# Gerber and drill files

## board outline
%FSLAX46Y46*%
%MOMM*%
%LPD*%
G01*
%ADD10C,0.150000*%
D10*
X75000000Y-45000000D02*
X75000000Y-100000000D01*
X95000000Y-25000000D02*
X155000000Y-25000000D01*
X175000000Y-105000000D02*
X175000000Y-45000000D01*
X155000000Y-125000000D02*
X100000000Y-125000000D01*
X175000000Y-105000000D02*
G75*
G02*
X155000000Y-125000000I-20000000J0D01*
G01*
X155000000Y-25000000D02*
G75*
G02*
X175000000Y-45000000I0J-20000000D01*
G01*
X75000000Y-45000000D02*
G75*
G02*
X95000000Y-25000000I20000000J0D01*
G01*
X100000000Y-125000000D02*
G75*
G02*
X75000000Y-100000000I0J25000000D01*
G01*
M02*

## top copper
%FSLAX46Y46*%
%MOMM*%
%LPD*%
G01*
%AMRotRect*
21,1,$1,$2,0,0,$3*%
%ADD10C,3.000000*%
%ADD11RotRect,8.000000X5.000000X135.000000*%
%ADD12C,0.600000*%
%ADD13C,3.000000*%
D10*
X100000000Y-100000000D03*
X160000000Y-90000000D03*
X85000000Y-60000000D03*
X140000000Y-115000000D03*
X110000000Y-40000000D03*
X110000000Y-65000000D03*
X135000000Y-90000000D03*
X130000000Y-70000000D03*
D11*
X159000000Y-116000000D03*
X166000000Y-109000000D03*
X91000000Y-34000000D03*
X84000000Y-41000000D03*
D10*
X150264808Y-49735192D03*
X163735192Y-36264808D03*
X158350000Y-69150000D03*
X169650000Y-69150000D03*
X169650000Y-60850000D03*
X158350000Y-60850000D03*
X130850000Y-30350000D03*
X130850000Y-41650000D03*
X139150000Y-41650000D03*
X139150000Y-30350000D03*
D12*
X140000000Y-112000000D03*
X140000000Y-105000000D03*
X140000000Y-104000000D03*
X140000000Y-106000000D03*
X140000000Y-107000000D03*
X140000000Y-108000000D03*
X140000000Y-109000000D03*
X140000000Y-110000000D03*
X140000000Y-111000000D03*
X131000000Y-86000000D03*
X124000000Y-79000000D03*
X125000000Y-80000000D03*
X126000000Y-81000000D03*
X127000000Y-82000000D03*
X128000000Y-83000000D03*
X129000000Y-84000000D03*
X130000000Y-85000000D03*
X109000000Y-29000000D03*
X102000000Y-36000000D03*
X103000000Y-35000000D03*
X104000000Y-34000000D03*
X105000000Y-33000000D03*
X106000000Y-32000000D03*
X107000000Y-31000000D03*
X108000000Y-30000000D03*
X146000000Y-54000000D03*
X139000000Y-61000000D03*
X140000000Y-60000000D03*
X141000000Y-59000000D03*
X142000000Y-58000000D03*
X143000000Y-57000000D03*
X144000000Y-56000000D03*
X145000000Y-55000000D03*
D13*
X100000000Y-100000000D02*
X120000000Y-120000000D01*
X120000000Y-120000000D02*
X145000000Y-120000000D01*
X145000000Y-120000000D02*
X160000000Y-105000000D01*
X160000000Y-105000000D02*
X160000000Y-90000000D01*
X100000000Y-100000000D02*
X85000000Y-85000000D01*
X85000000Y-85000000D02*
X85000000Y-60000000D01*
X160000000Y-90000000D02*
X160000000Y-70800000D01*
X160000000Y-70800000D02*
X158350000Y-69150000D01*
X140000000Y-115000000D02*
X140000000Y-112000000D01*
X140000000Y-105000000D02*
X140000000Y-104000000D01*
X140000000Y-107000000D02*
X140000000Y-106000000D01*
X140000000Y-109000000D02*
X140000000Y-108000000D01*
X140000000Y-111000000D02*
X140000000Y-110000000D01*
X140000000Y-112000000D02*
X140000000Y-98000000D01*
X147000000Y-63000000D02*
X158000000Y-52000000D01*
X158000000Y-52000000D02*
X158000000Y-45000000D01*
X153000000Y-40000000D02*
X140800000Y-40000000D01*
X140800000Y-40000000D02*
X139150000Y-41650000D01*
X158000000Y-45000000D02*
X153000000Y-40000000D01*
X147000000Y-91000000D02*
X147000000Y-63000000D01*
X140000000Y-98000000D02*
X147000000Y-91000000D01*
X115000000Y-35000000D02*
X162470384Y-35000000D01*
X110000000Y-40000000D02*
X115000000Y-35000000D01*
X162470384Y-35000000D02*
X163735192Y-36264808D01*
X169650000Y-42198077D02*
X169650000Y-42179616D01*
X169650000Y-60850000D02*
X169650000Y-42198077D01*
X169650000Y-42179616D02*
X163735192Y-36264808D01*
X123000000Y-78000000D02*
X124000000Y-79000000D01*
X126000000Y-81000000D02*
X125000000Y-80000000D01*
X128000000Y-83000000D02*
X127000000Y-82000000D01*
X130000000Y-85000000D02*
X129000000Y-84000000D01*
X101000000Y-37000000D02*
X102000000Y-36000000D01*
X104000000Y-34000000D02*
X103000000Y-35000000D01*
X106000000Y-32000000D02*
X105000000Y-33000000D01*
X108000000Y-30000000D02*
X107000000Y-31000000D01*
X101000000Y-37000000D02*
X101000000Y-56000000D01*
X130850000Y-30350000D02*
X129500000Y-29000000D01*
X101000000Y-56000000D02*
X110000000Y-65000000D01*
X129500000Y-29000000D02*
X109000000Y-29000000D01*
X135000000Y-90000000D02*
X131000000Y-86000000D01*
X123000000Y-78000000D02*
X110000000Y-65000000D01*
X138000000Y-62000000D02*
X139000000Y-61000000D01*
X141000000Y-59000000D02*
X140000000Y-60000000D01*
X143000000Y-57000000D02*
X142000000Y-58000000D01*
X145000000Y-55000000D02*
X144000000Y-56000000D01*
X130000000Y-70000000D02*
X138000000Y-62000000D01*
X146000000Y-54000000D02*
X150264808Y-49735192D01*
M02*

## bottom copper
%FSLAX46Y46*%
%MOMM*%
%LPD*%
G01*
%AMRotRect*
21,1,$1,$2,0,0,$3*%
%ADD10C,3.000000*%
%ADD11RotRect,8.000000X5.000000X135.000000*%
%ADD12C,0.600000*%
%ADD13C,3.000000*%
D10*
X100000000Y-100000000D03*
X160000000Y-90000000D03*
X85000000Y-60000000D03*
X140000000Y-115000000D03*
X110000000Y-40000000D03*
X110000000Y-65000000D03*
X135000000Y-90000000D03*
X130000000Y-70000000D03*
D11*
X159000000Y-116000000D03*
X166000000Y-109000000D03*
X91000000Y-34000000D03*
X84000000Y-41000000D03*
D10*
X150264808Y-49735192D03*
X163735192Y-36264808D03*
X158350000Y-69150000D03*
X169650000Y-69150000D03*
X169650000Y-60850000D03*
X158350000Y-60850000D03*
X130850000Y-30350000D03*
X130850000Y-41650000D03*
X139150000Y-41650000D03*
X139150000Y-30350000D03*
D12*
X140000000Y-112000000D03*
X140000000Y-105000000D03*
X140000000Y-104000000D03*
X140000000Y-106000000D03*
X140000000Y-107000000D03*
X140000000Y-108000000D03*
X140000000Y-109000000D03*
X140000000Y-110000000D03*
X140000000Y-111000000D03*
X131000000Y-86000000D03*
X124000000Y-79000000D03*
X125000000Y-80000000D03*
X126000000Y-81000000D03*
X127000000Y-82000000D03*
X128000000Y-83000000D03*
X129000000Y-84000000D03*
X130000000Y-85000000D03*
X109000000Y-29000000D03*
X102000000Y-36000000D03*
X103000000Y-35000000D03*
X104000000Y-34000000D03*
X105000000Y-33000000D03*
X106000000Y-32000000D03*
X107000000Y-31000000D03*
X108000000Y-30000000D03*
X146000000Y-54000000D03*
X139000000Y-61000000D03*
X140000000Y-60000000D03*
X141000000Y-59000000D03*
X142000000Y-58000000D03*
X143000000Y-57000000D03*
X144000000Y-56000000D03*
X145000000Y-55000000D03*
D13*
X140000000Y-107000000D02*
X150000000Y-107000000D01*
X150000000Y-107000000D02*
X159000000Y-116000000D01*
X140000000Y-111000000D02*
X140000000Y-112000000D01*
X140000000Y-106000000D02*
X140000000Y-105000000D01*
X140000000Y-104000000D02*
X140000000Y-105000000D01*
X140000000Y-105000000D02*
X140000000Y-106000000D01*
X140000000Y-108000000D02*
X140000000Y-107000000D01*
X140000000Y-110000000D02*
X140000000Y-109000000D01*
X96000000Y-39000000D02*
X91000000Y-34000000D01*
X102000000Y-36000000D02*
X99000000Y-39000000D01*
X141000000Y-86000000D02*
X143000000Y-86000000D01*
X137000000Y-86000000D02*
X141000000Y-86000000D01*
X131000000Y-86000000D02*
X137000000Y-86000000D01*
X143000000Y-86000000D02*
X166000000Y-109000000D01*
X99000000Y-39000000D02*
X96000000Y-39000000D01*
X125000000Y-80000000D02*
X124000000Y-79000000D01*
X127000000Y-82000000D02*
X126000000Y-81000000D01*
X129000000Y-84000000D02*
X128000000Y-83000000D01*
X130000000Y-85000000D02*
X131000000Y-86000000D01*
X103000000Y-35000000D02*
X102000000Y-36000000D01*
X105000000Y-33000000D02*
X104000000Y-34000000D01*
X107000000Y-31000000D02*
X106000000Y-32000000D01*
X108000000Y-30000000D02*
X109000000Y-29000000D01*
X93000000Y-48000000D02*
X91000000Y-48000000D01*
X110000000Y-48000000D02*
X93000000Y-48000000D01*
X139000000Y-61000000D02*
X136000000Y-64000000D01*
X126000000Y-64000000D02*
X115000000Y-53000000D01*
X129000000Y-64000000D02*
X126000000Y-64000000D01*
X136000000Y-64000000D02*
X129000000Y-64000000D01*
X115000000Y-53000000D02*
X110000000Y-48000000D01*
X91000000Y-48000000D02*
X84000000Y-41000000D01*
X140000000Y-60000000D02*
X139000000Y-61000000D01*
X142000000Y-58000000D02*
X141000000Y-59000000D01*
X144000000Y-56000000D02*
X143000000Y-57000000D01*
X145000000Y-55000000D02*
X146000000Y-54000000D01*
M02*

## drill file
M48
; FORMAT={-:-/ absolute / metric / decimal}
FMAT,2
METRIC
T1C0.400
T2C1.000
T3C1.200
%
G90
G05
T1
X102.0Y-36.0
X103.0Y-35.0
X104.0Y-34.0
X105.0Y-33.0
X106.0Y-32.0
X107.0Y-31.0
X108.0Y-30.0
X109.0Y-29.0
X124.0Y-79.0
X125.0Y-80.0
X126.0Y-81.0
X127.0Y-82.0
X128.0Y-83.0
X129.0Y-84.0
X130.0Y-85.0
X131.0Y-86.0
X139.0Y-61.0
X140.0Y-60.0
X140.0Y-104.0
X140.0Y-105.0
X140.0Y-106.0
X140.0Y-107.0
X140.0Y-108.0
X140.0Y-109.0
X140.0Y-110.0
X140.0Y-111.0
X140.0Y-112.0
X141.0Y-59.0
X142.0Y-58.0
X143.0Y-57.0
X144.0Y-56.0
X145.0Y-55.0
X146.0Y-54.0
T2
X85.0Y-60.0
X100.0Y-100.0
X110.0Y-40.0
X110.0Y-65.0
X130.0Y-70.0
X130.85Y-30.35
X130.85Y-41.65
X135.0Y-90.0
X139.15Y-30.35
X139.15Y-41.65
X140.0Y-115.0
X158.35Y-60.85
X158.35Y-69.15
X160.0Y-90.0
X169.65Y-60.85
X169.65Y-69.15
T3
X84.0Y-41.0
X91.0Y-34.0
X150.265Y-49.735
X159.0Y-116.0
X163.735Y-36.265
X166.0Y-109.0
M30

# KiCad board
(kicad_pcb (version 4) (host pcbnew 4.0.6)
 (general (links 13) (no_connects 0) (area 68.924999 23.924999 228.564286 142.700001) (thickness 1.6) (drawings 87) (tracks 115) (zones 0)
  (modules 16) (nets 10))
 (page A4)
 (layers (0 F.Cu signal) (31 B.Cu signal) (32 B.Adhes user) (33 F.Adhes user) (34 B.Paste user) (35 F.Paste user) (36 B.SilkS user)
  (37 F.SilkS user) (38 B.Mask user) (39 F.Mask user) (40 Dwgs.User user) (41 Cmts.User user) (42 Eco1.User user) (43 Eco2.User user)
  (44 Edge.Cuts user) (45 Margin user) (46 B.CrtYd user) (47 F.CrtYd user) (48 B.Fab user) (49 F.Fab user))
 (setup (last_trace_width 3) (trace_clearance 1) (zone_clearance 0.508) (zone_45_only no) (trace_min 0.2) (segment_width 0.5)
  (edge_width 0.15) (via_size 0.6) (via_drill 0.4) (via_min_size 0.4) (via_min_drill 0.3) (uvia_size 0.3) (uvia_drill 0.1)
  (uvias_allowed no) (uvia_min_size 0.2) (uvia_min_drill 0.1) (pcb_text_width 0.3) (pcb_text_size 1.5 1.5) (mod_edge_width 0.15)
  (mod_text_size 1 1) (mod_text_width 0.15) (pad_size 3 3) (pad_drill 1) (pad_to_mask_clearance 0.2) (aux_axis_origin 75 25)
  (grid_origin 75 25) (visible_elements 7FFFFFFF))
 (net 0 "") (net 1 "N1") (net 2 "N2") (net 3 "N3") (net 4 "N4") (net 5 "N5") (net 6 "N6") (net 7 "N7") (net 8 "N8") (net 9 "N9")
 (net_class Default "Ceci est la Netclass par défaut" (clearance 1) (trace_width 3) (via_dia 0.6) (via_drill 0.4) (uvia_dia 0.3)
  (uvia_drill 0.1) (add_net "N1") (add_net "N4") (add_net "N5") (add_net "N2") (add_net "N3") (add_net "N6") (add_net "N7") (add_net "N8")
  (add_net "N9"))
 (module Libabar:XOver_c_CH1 (layer F.Cu) (at 100 100)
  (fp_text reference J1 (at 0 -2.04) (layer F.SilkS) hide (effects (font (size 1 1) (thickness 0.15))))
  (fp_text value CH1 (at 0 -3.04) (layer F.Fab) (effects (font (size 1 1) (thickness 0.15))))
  (pad 1 thru_hole circle (at 0 0) (size 3 3) (drill 1) (layers *.Mask F.Cu) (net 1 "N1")))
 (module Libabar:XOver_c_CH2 (layer F.Cu) (at 160 90)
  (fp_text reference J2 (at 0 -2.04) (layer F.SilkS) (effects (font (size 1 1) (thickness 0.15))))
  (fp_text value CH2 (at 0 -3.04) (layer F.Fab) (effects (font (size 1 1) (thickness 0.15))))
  (pad 1 thru_hole circle (at 0 0) (size 3 3) (drill 1) (layers *.Mask F.Cu) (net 1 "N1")))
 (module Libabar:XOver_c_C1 (layer F.Cu) (at 85 60)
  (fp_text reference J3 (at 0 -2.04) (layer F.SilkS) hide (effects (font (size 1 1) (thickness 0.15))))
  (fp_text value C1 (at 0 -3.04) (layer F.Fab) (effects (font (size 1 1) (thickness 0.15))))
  (pad 1 thru_hole circle (at 0 0) (size 3 3) (drill 1) (layers *.Mask F.Cu) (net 1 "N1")))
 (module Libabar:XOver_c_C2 (layer F.Cu) (at 140 115)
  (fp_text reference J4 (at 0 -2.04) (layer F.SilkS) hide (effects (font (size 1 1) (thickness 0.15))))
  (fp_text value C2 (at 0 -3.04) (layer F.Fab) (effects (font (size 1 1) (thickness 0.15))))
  (pad 1 thru_hole circle (at 0 0) (size 3 3) (drill 1) (layers *.Mask F.Cu) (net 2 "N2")))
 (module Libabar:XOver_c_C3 (layer F.Cu) (at 110 40)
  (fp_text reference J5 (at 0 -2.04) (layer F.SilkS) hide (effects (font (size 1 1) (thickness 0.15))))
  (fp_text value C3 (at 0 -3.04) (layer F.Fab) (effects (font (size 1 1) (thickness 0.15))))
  (pad 1 thru_hole circle (at 0 0) (size 3 3) (drill 1) (layers *.Mask F.Cu) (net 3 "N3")))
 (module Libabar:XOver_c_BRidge (layer F.Cu) (at 110 65)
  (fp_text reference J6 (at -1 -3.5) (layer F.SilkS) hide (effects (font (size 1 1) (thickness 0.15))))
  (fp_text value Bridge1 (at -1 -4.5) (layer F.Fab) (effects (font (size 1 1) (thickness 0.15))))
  (pad 1 thru_hole circle (at 0 0) (size 3 3) (drill 1) (layers *.Mask F.Cu) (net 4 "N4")))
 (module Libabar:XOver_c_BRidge (layer F.Cu) (at 135 90)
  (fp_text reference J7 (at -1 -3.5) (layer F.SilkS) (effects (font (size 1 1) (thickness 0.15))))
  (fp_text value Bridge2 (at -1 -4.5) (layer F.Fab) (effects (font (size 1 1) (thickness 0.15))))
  (pad 1 thru_hole circle (at 0 0) (size 3 3) (drill 1) (layers *.Mask F.Cu) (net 4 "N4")))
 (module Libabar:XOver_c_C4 (layer F.Cu) (at 130 70)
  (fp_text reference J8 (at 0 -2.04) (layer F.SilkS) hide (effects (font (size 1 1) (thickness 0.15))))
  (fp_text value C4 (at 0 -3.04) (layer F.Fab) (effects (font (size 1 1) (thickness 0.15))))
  (pad 1 thru_hole circle (at 0 0) (size 3 3) (drill 1) (layers *.Mask F.Cu) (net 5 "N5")))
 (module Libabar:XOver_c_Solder (layer F.Cu) (at 159 116 135)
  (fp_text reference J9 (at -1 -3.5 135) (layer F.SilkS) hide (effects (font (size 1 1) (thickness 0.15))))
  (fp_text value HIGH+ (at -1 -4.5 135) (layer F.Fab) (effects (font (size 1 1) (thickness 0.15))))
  (pad 1 thru_hole rect (at 0 0 135) (size 8 5) (drill 1.2) (layers *.Cu *.Mask) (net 2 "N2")))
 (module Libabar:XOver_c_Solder (layer F.Cu) (at 166 109 135)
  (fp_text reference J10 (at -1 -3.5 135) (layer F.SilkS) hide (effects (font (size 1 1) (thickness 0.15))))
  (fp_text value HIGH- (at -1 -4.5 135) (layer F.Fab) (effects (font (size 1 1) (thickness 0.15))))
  (pad 1 thru_hole rect (at 0 0 135) (size 8 5) (drill 1.2) (layers *.Cu *.Mask) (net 4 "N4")))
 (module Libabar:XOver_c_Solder (layer F.Cu) (at 91 34 135)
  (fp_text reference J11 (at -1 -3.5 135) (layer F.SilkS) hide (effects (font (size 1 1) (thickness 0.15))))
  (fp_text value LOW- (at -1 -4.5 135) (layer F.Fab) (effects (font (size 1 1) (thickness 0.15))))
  (pad 1 thru_hole rect (at 0 0 135) (size 8 5) (drill 1.2) (layers *.Cu *.Mask) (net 4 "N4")))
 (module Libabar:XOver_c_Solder (layer F.Cu) (at 84 41 135)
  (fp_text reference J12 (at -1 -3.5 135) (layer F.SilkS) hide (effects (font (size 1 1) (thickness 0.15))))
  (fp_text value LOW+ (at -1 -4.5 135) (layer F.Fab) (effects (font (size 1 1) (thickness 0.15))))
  (pad 1 thru_hole rect (at 0 0 135) (size 8 5) (drill 1.2) (layers *.Cu *.Mask) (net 5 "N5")))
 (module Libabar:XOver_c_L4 (layer B.Cu) (at 157 43 225)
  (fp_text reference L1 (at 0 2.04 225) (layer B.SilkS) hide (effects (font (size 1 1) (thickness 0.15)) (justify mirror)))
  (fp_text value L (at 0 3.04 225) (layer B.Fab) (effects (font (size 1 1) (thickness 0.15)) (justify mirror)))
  (pad 1 thru_hole circle (at 9.525 0 225) (size 3 3) (drill 1.2) (layers *.Mask F.Cu) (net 5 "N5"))
  (pad 2 thru_hole circle (at -9.525 0 225) (size 3 3) (drill 1.2) (layers *.Mask F.Cu) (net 3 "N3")))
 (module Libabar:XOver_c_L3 (layer B.Cu) (at 164 65 180)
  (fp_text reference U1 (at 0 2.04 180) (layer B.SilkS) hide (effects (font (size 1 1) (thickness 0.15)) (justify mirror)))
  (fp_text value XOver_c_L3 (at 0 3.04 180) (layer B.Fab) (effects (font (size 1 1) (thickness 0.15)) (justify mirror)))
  (pad 1 thru_hole circle (at 5.65 -4.15 180) (size 3 3) (drill 1) (layers *.Mask F.Cu) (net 1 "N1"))
  (pad 2 thru_hole circle (at -5.65 -4.15 180) (size 3 3) (drill 1) (layers *.Mask F.Cu) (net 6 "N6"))
  (pad 3 thru_hole circle (at -5.65 4.15 180) (size 3 3) (drill 1) (layers *.Mask F.Cu) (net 3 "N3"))
  (pad 4 thru_hole circle (at 5.65 4.15 180) (size 3 3) (drill 1) (layers *.Mask F.Cu) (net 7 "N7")))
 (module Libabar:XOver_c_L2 (layer B.Cu) (at 135 36 90)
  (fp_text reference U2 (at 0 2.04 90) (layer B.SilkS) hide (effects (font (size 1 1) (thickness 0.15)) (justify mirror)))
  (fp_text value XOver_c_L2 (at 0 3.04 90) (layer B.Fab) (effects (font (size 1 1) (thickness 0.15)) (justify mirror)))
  (pad 1 thru_hole circle (at 5.65 -4.15 90) (size 3 3) (drill 1) (layers *.Mask F.Cu) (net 4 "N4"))
  (pad 2 thru_hole circle (at -5.65 -4.15 90) (size 3 3) (drill 1) (layers *.Mask F.Cu) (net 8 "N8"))
  (pad 3 thru_hole circle (at -5.65 4.15 90) (size 3 3) (drill 1) (layers *.Mask F.Cu) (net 2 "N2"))
  (pad 4 thru_hole circle (at 5.65 4.15 90) (size 3 3) (drill 1) (layers *.Mask F.Cu) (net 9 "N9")))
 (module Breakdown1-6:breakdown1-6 (layer F.Cu) (at 91 109 135)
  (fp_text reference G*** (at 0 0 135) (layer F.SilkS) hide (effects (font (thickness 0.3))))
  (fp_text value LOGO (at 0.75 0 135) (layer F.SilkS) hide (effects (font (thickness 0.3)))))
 (gr_line (start 75 45) (end 75 100) (angle 90) (layer Edge.Cuts) (width 0.15))
 (gr_line (start 95 25) (end 155 25) (angle 90) (layer Edge.Cuts) (width 0.15))
 (gr_line (start 175 105) (end 175 45) (angle 90) (layer Edge.Cuts) (width 0.15))
 (gr_line (start 155 125) (end 100 125) (angle 90) (layer Edge.Cuts) (width 0.15))
 (gr_arc (start 155 105) (end 175 105) (angle 90) (layer Edge.Cuts) (width 0.15))
 (gr_arc (start 155 45) (end 155 25) (angle 90) (layer Edge.Cuts) (width 0.15))
 (gr_arc (start 95 45) (end 75 45) (angle 90) (layer Edge.Cuts) (width 0.15))
 (gr_arc (start 100 100) (end 100 125) (angle 90) (layer Edge.Cuts) (width 0.15))
 (segment (start 100 100) (end 120 120) (width 3) (layer F.Cu) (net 1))
 (segment (start 120 120) (end 145 120) (width 3) (layer F.Cu) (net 1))
 (segment (start 145 120) (end 160 105) (width 3) (layer F.Cu) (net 1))
 (segment (start 160 105) (end 160 90) (width 3) (layer F.Cu) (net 1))
 (segment (start 100 100) (end 85 85) (width 3) (layer F.Cu) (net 1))
 (segment (start 85 85) (end 85 60) (width 3) (layer F.Cu) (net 1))
 (segment (start 160 90) (end 160 70.8) (width 3) (layer F.Cu) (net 1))
 (segment (start 160 70.8) (end 158.35 69.15) (width 3) (layer F.Cu) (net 1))
 (segment (start 140 107) (end 150 107) (width 3) (layer B.Cu) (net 2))
 (segment (start 150 107) (end 159 116) (width 3) (layer B.Cu) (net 2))
 (via (at 140 112) (size 0.6) (drill 0.4) (layers F.Cu B.Cu) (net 2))
 (segment (start 140 111) (end 140 112) (width 3) (layer B.Cu) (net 2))
 (segment (start 140 115) (end 140 112) (width 3) (layer F.Cu) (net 2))
 (segment (start 140 106) (end 140 105) (width 3) (layer B.Cu) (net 2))
 (via (at 140 105) (size 0.6) (drill 0.4) (layers F.Cu B.Cu) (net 2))
 (segment (start 140 105) (end 140 104) (width 3) (layer F.Cu) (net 2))
 (via (at 140 104) (size 0.6) (drill 0.4) (layers F.Cu B.Cu) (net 2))
 (segment (start 140 104) (end 140 105) (width 3) (layer B.Cu) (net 2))
 (segment (start 140 105) (end 140 106) (width 3) (layer B.Cu) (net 2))
 (via (at 140 106) (size 0.6) (drill 0.4) (layers F.Cu B.Cu) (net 2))
 (segment (start 140 107) (end 140 106) (width 3) (layer F.Cu) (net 2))
 (via (at 140 107) (size 0.6) (drill 0.4) (layers F.Cu B.Cu) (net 2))
 (segment (start 140 108) (end 140 107) (width 3) (layer B.Cu) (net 2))
 (via (at 140 108) (size 0.6) (drill 0.4) (layers F.Cu B.Cu) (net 2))
 (segment (start 140 109) (end 140 108) (width 3) (layer F.Cu) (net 2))
 (via (at 140 109) (size 0.6) (drill 0.4) (layers F.Cu B.Cu) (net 2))
 (segment (start 140 110) (end 140 109) (width 3) (layer B.Cu) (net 2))
 (via (at 140 110) (size 0.6) (drill 0.4) (layers F.Cu B.Cu) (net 2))
 (segment (start 140 111) (end 140 110) (width 3) (layer F.Cu) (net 2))
 (via (at 140 111) (size 0.6) (drill 0.4) (layers F.Cu B.Cu) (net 2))
 (segment (start 140 112) (end 140 98) (width 3) (layer F.Cu) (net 2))
 (segment (start 147 63) (end 158 52) (width 3) (layer F.Cu) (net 2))
 (segment (start 158 52) (end 158 45) (width 3) (layer F.Cu) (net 2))
 (segment (start 153 40) (end 140.8 40) (width 3) (layer F.Cu) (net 2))
 (segment (start 140.8 40) (end 139.15 41.65) (width 3) (layer F.Cu) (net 2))
 (segment (start 158 45) (end 153 40) (width 3) (layer F.Cu) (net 2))
 (segment (start 147 91) (end 147 63) (width 3) (layer F.Cu) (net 2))
 (segment (start 140 98) (end 147 91) (width 3) (layer F.Cu) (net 2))
 (segment (start 115 35) (end 162.470384 35) (width 3) (layer F.Cu) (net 3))
 (segment (start 110 40) (end 115 35) (width 3) (layer F.Cu) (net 3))
 (segment (start 162.470384 35) (end 163.735192 36.264808) (width 3) (layer F.Cu) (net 3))
 (segment (start 169.65 42.198077) (end 169.65 42.179616) (width 3) (layer F.Cu) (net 3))
 (segment (start 169.65 60.85) (end 169.65 42.198077) (width 3) (layer F.Cu) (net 3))
 (segment (start 169.65 42.179616) (end 163.735192 36.264808) (width 3) (layer F.Cu) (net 3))
 (segment (start 96 39) (end 91 34) (width 3) (layer B.Cu) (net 4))
 (segment (start 102 36) (end 99 39) (width 3) (layer B.Cu) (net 4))
 (segment (start 141 86) (end 143 86) (width 3) (layer B.Cu) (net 4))
 (segment (start 137 86) (end 141 86) (width 3) (layer B.Cu) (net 4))
 (segment (start 131 86) (end 137 86) (width 3) (layer B.Cu) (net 4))
 (segment (start 143 86) (end 166 109) (width 3) (layer B.Cu) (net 4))
 (segment (start 99 39) (end 96 39) (width 3) (layer B.Cu) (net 4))
 (via (at 131 86) (size 0.6) (drill 0.4) (layers F.Cu B.Cu) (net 4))
 (segment (start 123 78) (end 124 79) (width 3) (layer F.Cu) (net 4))
 (via (at 124 79) (size 0.6) (drill 0.4) (layers F.Cu B.Cu) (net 4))
 (segment (start 125 80) (end 124 79) (width 3) (layer B.Cu) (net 4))
 (via (at 125 80) (size 0.6) (drill 0.4) (layers F.Cu B.Cu) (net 4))
 (segment (start 126 81) (end 125 80) (width 3) (layer F.Cu) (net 4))
 (via (at 126 81) (size 0.6) (drill 0.4) (layers F.Cu B.Cu) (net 4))
 (segment (start 127 82) (end 126 81) (width 3) (layer B.Cu) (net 4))
 (via (at 127 82) (size 0.6) (drill 0.4) (layers F.Cu B.Cu) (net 4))
 (segment (start 128 83) (end 127 82) (width 3) (layer F.Cu) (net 4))
 (via (at 128 83) (size 0.6) (drill 0.4) (layers F.Cu B.Cu) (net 4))
 (segment (start 129 84) (end 128 83) (width 3) (layer B.Cu) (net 4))
 (via (at 129 84) (size 0.6) (drill 0.4) (layers F.Cu B.Cu) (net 4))
 (segment (start 130 85) (end 129 84) (width 3) (layer F.Cu) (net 4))
 (via (at 130 85) (size 0.6) (drill 0.4) (layers F.Cu B.Cu) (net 4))
 (segment (start 130 85) (end 131 86) (width 3) (layer B.Cu) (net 4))
 (via (at 109 29) (size 0.6) (drill 0.4) (layers F.Cu B.Cu) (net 4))
 (segment (start 101 37) (end 102 36) (width 3) (layer F.Cu) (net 4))
 (via (at 102 36) (size 0.6) (drill 0.4) (layers F.Cu B.Cu) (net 4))
 (segment (start 103 35) (end 102 36) (width 3) (layer B.Cu) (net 4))
 (via (at 103 35) (size 0.6) (drill 0.4) (layers F.Cu B.Cu) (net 4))
 (segment (start 104 34) (end 103 35) (width 3) (layer F.Cu) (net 4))
 (via (at 104 34) (size 0.6) (drill 0.4) (layers F.Cu B.Cu) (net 4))
 (segment (start 105 33) (end 104 34) (width 3) (layer B.Cu) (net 4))
 (via (at 105 33) (size 0.6) (drill 0.4) (layers F.Cu B.Cu) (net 4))
 (segment (start 106 32) (end 105 33) (width 3) (layer F.Cu) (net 4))
 (via (at 106 32) (size 0.6) (drill 0.4) (layers F.Cu B.Cu) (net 4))
 (segment (start 107 31) (end 106 32) (width 3) (layer B.Cu) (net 4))
 (via (at 107 31) (size 0.6) (drill 0.4) (layers F.Cu B.Cu) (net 4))
 (segment (start 108 30) (end 107 31) (width 3) (layer F.Cu) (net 4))
 (via (at 108 30) (size 0.6) (drill 0.4) (layers F.Cu B.Cu) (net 4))
 (segment (start 108 30) (end 109 29) (width 3) (layer B.Cu) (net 4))
 (segment (start 101 37) (end 101 56) (width 3) (layer F.Cu) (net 4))
 (segment (start 130.85 30.35) (end 129.5 29) (width 3) (layer F.Cu) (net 4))
 (segment (start 101 56) (end 110 65) (width 3) (layer F.Cu) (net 4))
 (segment (start 129.5 29) (end 109 29) (width 3) (layer F.Cu) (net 4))
 (segment (start 135 90) (end 131 86) (width 3) (layer F.Cu) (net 4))
 (segment (start 123 78) (end 110 65) (width 3) (layer F.Cu) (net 4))
 (segment (start 93 48) (end 91 48) (width 3) (layer B.Cu) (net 5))
 (segment (start 110 48) (end 93 48) (width 3) (layer B.Cu) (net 5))
 (segment (start 139 61) (end 136 64) (width 3) (layer B.Cu) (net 5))
 (segment (start 126 64) (end 115 53) (width 3) (layer B.Cu) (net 5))
 (segment (start 129 64) (end 126 64) (width 3) (layer B.Cu) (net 5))
 (segment (start 136 64) (end 129 64) (width 3) (layer B.Cu) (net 5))
 (segment (start 115 53) (end 110 48) (width 3) (layer B.Cu) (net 5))
 (segment (start 91 48) (end 84 41) (width 3) (layer B.Cu) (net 5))
 (via (at 146 54) (size 0.6) (drill 0.4) (layers F.Cu B.Cu) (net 5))
 (segment (start 138 62) (end 139 61) (width 3) (layer F.Cu) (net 5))
 (via (at 139 61) (size 0.6) (drill 0.4) (layers F.Cu B.Cu) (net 5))
 (segment (start 140 60) (end 139 61) (width 3) (layer B.Cu) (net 5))
 (via (at 140 60) (size 0.6) (drill 0.4) (layers F.Cu B.Cu) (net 5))
 (segment (start 141 59) (end 140 60) (width 3) (layer F.Cu) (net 5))
 (via (at 141 59) (size 0.6) (drill 0.4) (layers F.Cu B.Cu) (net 5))
 (segment (start 142 58) (end 141 59) (width 3) (layer B.Cu) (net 5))
 (via (at 142 58) (size 0.6) (drill 0.4) (layers F.Cu B.Cu) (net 5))
 (segment (start 143 57) (end 142 58) (width 3) (layer F.Cu) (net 5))
 (via (at 143 57) (size 0.6) (drill 0.4) (layers F.Cu B.Cu) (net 5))
 (segment (start 144 56) (end 143 57) (width 3) (layer B.Cu) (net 5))
 (via (at 144 56) (size 0.6) (drill 0.4) (layers F.Cu B.Cu) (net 5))
 (segment (start 145 55) (end 144 56) (width 3) (layer F.Cu) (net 5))
 (via (at 145 55) (size 0.6) (drill 0.4) (layers F.Cu B.Cu) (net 5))
 (segment (start 145 55) (end 146 54) (width 3) (layer B.Cu) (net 5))
 (segment (start 130 70) (end 138 62) (width 3) (layer F.Cu) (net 5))
 (segment (start 146 54) (end 150.264808 49.735192) (width 3) (layer F.Cu) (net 5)))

